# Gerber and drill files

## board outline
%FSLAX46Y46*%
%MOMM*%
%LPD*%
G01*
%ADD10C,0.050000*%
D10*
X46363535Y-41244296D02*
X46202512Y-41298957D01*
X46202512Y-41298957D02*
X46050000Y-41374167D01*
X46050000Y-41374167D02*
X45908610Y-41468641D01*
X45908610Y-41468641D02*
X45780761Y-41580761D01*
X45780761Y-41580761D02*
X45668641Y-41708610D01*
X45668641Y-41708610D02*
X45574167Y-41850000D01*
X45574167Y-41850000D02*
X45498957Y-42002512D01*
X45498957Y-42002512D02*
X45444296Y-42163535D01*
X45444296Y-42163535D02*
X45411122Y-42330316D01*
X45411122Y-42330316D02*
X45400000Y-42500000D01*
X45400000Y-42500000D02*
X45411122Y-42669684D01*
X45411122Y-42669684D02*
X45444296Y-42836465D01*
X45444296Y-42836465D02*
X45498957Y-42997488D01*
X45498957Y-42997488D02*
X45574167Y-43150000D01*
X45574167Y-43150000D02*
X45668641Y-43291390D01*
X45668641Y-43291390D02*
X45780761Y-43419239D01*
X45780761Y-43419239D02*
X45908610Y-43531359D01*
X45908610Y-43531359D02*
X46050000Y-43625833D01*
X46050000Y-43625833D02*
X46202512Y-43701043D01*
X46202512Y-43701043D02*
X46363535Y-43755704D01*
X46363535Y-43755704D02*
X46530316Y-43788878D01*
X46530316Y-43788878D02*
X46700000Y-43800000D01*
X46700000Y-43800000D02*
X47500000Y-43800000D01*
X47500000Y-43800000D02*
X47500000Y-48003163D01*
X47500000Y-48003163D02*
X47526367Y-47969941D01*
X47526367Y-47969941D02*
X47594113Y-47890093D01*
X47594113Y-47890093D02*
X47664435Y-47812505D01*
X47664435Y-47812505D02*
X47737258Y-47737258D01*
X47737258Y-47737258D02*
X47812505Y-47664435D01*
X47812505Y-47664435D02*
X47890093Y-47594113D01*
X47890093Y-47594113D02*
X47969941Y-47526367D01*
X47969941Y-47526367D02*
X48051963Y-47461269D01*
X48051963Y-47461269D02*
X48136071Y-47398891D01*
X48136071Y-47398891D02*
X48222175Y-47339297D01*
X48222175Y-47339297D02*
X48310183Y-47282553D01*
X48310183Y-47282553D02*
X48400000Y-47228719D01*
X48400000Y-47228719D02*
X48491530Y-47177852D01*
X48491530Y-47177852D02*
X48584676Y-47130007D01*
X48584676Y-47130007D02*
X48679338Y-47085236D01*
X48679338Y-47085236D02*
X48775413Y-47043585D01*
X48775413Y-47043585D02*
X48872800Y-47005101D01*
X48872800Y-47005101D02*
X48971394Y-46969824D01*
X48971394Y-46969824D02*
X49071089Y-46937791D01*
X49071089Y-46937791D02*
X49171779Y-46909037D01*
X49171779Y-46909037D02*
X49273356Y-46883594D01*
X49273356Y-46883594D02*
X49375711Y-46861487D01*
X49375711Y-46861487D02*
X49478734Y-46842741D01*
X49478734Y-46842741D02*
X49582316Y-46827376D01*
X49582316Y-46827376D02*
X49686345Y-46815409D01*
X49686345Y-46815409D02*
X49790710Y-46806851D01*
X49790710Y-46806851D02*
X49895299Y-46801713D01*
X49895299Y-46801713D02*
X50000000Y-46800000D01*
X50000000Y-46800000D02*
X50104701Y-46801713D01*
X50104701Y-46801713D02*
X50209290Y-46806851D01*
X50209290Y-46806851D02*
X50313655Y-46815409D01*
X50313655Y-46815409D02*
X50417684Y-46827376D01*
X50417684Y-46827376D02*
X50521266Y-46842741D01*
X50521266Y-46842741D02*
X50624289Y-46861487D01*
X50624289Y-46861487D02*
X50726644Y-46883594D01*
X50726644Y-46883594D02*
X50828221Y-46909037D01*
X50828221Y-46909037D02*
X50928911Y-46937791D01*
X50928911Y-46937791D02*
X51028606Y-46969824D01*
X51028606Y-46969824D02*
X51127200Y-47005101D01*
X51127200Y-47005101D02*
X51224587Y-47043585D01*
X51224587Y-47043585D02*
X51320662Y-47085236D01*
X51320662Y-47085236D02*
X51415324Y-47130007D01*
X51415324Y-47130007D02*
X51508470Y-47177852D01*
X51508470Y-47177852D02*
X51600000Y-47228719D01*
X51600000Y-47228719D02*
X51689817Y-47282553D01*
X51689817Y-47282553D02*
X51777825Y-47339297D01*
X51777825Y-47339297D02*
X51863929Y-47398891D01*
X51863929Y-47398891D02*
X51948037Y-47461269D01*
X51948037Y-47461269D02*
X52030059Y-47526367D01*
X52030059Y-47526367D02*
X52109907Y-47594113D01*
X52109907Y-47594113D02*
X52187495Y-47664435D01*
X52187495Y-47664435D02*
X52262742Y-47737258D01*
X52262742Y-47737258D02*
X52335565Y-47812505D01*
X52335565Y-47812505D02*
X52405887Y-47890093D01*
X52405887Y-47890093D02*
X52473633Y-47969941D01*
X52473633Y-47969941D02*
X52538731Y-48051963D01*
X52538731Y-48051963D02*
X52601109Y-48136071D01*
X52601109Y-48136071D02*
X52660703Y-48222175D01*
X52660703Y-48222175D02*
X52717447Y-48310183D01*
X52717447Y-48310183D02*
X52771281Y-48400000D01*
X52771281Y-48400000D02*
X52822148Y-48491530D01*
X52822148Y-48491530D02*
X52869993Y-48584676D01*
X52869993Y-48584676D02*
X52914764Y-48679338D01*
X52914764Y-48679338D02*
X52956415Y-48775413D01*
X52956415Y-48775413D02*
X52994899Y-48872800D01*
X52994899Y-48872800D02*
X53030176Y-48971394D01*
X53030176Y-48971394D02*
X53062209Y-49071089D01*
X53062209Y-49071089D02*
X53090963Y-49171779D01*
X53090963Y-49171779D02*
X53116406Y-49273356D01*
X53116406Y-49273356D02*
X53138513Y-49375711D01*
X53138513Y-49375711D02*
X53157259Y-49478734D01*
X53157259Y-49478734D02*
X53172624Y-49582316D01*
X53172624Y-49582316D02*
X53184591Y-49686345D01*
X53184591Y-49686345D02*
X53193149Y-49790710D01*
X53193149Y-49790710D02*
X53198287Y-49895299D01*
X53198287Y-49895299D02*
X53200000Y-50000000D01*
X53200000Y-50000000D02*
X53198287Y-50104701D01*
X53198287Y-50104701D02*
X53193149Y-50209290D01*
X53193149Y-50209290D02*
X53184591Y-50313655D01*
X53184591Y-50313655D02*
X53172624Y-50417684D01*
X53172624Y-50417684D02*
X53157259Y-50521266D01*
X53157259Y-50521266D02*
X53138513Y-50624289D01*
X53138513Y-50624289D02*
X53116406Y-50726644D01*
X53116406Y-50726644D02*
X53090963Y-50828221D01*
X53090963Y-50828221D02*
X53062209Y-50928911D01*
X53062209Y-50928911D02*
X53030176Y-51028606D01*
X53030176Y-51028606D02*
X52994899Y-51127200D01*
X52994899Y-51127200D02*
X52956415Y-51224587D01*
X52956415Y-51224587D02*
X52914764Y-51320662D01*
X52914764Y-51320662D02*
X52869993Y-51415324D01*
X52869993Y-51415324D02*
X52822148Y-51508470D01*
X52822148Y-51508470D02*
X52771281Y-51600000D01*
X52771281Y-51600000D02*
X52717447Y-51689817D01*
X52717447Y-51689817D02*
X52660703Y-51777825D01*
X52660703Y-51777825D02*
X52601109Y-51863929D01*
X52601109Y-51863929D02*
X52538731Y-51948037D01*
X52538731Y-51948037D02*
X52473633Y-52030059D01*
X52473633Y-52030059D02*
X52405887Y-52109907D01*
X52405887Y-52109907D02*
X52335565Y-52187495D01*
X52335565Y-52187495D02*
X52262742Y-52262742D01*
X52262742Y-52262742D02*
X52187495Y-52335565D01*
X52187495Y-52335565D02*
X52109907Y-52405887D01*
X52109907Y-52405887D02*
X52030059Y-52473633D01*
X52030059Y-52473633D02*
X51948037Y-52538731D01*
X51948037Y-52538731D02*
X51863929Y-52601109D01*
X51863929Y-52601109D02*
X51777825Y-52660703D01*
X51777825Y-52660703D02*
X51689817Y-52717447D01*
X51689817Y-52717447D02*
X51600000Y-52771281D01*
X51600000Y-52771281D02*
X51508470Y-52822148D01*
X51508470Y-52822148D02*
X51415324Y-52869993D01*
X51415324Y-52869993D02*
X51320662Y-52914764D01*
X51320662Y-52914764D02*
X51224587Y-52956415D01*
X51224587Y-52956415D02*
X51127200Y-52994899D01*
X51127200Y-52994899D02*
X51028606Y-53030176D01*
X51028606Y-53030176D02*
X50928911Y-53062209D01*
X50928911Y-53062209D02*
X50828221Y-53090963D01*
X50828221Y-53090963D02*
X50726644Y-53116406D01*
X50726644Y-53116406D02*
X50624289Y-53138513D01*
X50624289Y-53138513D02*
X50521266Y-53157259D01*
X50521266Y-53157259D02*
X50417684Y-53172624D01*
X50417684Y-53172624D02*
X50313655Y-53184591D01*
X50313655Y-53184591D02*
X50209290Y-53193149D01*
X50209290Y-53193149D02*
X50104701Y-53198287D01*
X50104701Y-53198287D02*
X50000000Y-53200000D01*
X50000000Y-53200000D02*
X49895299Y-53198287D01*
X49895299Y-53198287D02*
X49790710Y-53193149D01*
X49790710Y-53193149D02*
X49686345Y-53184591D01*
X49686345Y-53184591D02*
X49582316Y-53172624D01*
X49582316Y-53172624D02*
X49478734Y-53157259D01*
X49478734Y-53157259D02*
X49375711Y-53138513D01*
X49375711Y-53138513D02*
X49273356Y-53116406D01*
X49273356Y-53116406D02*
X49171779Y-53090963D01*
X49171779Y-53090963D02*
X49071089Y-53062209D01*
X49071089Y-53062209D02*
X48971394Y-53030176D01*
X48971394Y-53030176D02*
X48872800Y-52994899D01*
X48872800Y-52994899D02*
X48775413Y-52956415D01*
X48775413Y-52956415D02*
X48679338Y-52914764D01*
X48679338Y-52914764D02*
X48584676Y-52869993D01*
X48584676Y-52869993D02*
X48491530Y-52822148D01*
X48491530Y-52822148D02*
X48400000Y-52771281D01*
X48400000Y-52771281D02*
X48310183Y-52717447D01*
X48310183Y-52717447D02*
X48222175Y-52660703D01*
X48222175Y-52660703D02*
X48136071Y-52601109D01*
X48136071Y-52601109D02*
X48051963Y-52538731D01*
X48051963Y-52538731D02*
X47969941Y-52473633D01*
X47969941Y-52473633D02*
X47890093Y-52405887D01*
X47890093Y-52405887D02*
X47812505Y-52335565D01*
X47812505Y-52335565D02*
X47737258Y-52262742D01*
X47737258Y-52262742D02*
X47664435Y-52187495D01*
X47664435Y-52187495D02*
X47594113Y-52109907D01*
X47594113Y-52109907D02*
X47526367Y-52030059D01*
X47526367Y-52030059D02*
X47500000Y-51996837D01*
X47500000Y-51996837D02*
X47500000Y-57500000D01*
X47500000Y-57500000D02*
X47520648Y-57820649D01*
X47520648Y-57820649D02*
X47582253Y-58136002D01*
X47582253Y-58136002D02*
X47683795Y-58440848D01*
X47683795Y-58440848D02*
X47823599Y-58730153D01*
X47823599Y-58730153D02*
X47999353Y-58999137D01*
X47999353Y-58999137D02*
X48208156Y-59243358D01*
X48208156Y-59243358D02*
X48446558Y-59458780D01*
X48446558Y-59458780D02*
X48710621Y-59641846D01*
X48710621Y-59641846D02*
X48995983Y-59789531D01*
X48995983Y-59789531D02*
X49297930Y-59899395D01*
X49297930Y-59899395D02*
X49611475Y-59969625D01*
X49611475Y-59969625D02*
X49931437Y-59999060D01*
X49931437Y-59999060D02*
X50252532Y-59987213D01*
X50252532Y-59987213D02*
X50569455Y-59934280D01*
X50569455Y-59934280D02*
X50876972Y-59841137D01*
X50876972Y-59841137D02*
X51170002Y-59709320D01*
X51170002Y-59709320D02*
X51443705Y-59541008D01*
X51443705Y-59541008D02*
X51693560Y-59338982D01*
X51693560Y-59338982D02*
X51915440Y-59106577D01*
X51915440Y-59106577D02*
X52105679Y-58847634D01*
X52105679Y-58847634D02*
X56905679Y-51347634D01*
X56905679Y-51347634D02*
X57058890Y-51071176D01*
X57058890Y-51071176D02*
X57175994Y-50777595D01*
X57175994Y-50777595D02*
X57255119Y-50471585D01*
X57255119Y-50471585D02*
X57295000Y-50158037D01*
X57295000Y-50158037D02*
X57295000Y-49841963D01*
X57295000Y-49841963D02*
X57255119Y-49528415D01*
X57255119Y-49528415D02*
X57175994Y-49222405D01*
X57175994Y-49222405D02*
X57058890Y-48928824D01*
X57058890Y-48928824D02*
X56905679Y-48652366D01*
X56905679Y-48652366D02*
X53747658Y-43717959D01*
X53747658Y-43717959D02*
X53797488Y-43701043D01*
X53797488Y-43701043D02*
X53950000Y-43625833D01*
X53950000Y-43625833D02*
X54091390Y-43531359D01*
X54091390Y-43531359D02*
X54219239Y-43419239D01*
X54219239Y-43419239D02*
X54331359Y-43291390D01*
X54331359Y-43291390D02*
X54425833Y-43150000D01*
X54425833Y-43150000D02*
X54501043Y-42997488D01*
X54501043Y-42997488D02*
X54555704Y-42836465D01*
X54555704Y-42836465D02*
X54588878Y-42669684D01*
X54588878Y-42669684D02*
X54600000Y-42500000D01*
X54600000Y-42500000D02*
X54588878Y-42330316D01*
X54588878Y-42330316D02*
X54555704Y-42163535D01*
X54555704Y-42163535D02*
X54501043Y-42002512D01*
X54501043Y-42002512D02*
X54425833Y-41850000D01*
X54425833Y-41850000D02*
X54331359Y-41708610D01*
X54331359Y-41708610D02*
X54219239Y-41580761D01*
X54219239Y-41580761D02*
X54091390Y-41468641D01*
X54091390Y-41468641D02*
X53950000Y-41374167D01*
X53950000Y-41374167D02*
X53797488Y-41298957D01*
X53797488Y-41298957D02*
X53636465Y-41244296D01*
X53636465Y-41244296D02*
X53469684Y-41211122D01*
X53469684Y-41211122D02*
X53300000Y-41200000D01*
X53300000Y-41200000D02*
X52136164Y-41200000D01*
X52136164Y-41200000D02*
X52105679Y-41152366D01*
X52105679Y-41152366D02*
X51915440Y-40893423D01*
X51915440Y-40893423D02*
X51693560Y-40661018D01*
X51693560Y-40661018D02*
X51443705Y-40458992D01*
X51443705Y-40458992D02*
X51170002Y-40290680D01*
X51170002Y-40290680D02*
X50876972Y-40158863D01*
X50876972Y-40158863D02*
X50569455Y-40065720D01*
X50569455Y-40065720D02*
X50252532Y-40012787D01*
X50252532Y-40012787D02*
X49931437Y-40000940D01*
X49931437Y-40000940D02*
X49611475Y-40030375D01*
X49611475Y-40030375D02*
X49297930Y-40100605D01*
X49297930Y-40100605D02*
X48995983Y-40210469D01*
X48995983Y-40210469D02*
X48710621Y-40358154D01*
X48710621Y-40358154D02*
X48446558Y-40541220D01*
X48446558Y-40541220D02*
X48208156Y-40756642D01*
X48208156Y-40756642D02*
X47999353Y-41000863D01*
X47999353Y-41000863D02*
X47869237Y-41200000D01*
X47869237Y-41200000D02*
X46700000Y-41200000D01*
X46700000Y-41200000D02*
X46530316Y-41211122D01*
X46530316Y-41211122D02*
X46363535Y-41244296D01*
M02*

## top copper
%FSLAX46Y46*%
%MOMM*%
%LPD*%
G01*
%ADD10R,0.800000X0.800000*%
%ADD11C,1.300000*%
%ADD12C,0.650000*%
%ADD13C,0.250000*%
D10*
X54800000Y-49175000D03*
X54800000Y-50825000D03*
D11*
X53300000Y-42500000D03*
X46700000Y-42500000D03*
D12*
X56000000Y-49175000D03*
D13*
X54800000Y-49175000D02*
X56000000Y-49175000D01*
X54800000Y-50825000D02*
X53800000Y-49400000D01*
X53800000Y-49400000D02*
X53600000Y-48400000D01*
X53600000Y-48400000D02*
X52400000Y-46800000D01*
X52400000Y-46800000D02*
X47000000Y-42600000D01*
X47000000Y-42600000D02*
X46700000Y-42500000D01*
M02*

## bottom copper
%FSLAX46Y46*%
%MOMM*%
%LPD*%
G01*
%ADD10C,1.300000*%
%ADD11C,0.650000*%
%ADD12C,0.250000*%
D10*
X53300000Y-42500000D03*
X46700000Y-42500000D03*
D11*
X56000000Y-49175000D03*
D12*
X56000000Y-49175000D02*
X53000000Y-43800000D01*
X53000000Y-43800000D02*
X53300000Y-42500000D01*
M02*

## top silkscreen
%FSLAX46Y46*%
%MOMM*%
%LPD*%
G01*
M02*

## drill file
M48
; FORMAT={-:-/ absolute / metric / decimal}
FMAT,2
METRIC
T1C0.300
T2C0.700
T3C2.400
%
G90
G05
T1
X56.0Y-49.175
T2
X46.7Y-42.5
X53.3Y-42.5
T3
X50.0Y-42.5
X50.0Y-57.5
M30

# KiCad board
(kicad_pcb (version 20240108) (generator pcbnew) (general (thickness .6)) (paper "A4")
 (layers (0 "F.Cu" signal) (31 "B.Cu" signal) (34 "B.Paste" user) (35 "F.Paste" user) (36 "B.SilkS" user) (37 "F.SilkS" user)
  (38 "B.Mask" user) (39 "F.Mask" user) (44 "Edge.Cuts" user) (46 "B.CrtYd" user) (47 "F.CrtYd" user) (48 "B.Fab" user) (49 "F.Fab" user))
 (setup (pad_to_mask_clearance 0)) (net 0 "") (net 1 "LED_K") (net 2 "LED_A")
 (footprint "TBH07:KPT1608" (layer "F.Cu") (at 54.8 50)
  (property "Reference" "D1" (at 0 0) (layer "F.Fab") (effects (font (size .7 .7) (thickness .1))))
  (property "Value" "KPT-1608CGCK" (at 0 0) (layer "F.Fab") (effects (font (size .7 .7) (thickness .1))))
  (pad "1" smd rect (at 0 -.825) (size .8 .8) (layers "F.Cu" "F.Paste" "F.Mask") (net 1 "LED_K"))
  (pad "2" smd rect (at 0 .825) (size .8 .8) (layers "F.Cu" "F.Paste" "F.Mask") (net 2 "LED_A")))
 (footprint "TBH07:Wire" (layer "F.Cu") (at 53.3 42.5)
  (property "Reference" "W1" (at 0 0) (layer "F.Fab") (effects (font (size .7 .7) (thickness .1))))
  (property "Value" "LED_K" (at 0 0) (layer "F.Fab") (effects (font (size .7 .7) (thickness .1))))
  (pad "1" thru_hole circle (at 0 0) (size 1.3 1.3) (drill .7) (layers "*.Cu" "*.Mask") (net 1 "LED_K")))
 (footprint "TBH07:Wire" (layer "F.Cu") (at 46.7 42.5)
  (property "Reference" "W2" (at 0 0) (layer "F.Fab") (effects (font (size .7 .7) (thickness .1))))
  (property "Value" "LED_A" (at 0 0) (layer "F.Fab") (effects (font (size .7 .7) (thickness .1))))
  (pad "1" thru_hole circle (at 0 0) (size 1.3 1.3) (drill .7) (layers "*.Cu" "*.Mask") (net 2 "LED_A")))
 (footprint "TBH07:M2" (layer "F.Cu") (at 50 42.5)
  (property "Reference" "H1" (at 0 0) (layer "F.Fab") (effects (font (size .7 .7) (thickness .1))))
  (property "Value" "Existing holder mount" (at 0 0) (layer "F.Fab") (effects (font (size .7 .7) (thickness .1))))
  (pad "" np_thru_hole circle (at 0 0) (size 2.4 2.4) (drill 2.4) (layers "*.Cu" "*.Mask")))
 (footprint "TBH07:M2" (layer "F.Cu") (at 50 57.5)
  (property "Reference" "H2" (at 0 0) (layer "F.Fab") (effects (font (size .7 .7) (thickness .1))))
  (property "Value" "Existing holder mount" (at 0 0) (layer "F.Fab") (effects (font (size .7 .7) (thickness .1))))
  (pad "" np_thru_hole circle (at 0 0) (size 2.4 2.4) (drill 2.4) (layers "*.Cu" "*.Mask")))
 (segment (start 54.8 49.175) (end 56 49.175) (width .25) (layer "F.Cu") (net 1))
 (via (at 56 49.175) (size .65) (drill .3) (layers "F.Cu" "B.Cu") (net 1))
 (segment (start 56 49.175) (end 53.0 43.8) (width .25) (layer "B.Cu") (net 1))
 (segment (start 53.0 43.8) (end 53.3 42.5) (width .25) (layer "B.Cu") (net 1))
 (segment (start 54.8 50.825) (end 53.8 49.4) (width .25) (layer "F.Cu") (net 2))
 (segment (start 53.8 49.4) (end 53.6 48.4) (width .25) (layer "F.Cu") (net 2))
 (segment (start 53.6 48.4) (end 52.4 46.8) (width .25) (layer "F.Cu") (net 2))
 (segment (start 52.4 46.8) (end 47.0 42.6) (width .25) (layer "F.Cu") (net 2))
 (segment (start 47.0 42.6) (end 46.7 42.5) (width .25) (layer "F.Cu") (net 2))
 (gr_line (start 46.363535241366726 41.24429642582421) (end 46.20251153792538 41.29895660773533) (stroke (width .05) (type default))
  (layer "Edge.Cuts"))
 (gr_line (start 46.20251153792538 41.29895660773533) (end 46.05 41.37416697508023) (stroke (width .05) (type default)) (layer "Edge.Cuts"))
 (gr_line (start 46.05 41.37416697508023) (end 45.908610142288666 41.46864065762139) (stroke (width .05) (type default)) (layer "Edge.Cuts"))
 (gr_line (start 45.908610142288666 41.46864065762139) (end 45.78076118445749 41.58076118445749) (stroke (width .05) (type default))
  (layer "Edge.Cuts"))
 (gr_line (start 45.78076118445749 41.58076118445749) (end 45.668640657621395 41.70861014228866) (stroke (width .05) (type default))
  (layer "Edge.Cuts"))
 (gr_line (start 45.668640657621395 41.70861014228866) (end 45.57416697508023 41.85) (stroke (width .05) (type default)) (layer "Edge.Cuts"))
 (gr_line (start 45.57416697508023 41.85) (end 45.49895660773532 42.002511537925386) (stroke (width .05) (type default)) (layer "Edge.Cuts"))
 (gr_line (start 45.49895660773532 42.002511537925386) (end 45.44429642582421 42.16353524136672) (stroke (width .05) (type default))
  (layer "Edge.Cuts"))
 (gr_line (start 45.44429642582421 42.16353524136672) (end 45.411121680214045 42.330315950113935) (stroke (width .05) (type default))
  (layer "Edge.Cuts"))
 (gr_line (start 45.411121680214045 42.330315950113935) (end 45.4 42.5) (stroke (width .05) (type default)) (layer "Edge.Cuts"))
 (gr_line (start 45.4 42.5) (end 45.411121680214045 42.669684049886065) (stroke (width .05) (type default)) (layer "Edge.Cuts"))
 (gr_line (start 45.411121680214045 42.669684049886065) (end 45.44429642582421 42.83646475863328) (stroke (width .05) (type default))
  (layer "Edge.Cuts"))
 (gr_line (start 45.44429642582421 42.83646475863328) (end 45.49895660773532 42.997488462074614) (stroke (width .05) (type default))
  (layer "Edge.Cuts"))
 (gr_line (start 45.49895660773532 42.997488462074614) (end 45.57416697508023 43.15) (stroke (width .05) (type default)) (layer "Edge.Cuts"))
 (gr_line (start 45.57416697508023 43.15) (end 45.668640657621395 43.29138985771134) (stroke (width .05) (type default)) (layer "Edge.Cuts"))
 (gr_line (start 45.668640657621395 43.29138985771134) (end 45.78076118445749 43.41923881554251) (stroke (width .05) (type default))
  (layer "Edge.Cuts"))
 (gr_line (start 45.78076118445749 43.41923881554251) (end 45.908610142288666 43.53135934237861) (stroke (width .05) (type default))
  (layer "Edge.Cuts"))
 (gr_line (start 45.908610142288666 43.53135934237861) (end 46.05 43.62583302491977) (stroke (width .05) (type default)) (layer "Edge.Cuts"))
 (gr_line (start 46.05 43.62583302491977) (end 46.20251153792538 43.70104339226467) (stroke (width .05) (type default)) (layer "Edge.Cuts"))
 (gr_line (start 46.20251153792538 43.70104339226467) (end 46.363535241366726 43.75570357417579) (stroke (width .05) (type default))
  (layer "Edge.Cuts"))
 (gr_line (start 46.363535241366726 43.75570357417579) (end 46.53031595011393 43.78887831978595) (stroke (width .05) (type default))
  (layer "Edge.Cuts"))
 (gr_line (start 46.53031595011393 43.78887831978595) (end 46.7 43.8) (stroke (width .05) (type default)) (layer "Edge.Cuts"))
 (gr_line (start 46.7 43.8) (end 47.5 43.8) (stroke (width .05) (type default)) (layer "Edge.Cuts"))
 (gr_line (start 47.5 43.8) (end 47.5 48.00316310634037) (stroke (width .05) (type default)) (layer "Edge.Cuts"))
 (gr_line (start 47.5 48.00316310634037) (end 47.52636654923924 47.969941490676334) (stroke (width .05) (type default)) (layer "Edge.Cuts"))
 (gr_line (start 47.52636654923924 47.969941490676334) (end 47.59411261606727 47.89009339167978) (stroke (width .05) (type default))
  (layer "Edge.Cuts"))
 (gr_line (start 47.59411261606727 47.89009339167978) (end 47.66443496736693 47.812504633526814) (stroke (width .05) (type default))
  (layer "Edge.Cuts"))
 (gr_line (start 47.66443496736693 47.812504633526814) (end 47.737258300203045 47.737258300203045) (stroke (width .05) (type default))
  (layer "Edge.Cuts"))
 (gr_line (start 47.737258300203045 47.737258300203045) (end 47.812504633526814 47.66443496736692) (stroke (width .05) (type default))
  (layer "Edge.Cuts"))
 (gr_line (start 47.812504633526814 47.66443496736692) (end 47.890093391679784 47.59411261606727) (stroke (width .05) (type default))
  (layer "Edge.Cuts"))
 (gr_line (start 47.890093391679784 47.59411261606727) (end 47.969941490676334 47.52636654923924) (stroke (width .05) (type default))
  (layer "Edge.Cuts"))
 (gr_line (start 47.969941490676334 47.52636654923924) (end 48.0519634271721 47.461269311068044) (stroke (width .05) (type default))
  (layer "Edge.Cuts"))
 (gr_line (start 48.0519634271721 47.461269311068044) (end 48.13607137002303 47.39889060930683) (stroke (width .05) (type default))
  (layer "Edge.Cuts"))
 (gr_line (start 48.13607137002303 47.39889060930683) (end 48.22217525433727 47.33929724063186) (stroke (width .05) (type default))
  (layer "Edge.Cuts"))
 (gr_line (start 48.22217525433727 47.33929724063186) (end 48.31018287791882 47.28255301911495) (stroke (width .05) (type default))
  (layer "Edge.Cuts"))
 (gr_line (start 48.31018287791882 47.28255301911495) (end 48.4 47.2287187078898) (stroke (width .05) (type default)) (layer "Edge.Cuts"))
 (gr_line (start 48.4 47.2287187078898) (end 48.49153044215681 47.17785195408526) (stroke (width .05) (type default)) (layer "Edge.Cuts"))
 (gr_line (start 48.49153044215681 47.17785195408526) (end 48.584676191299195 47.1300072270954) (stroke (width .05) (type default))
  (layer "Edge.Cuts"))
 (gr_line (start 48.584676191299195 47.1300072270954) (end 48.679337504625934 47.08523576025224) (stroke (width .05) (type default))
  (layer "Edge.Cuts"))
 (gr_line (start 48.679337504625934 47.08523576025224) (end 48.77541301643171 47.04358549596388) (stroke (width .05) (type default))
  (layer "Edge.Cuts"))
 (gr_line (start 48.77541301643171 47.04358549596388) (end 48.87279984665205 47.00510103437656) (stroke (width .05) (type default))
  (layer "Edge.Cuts"))
 (gr_line (start 48.87279984665205 47.00510103437656) (end 48.97139371102988 46.969823585615664) (stroke (width .05) (type default))
  (layer "Edge.Cuts"))
 (gr_line (start 48.97139371102988 46.969823585615664) (end 49.07108903278572 46.937790925656934) (stroke (width .05) (type default))
  (layer "Edge.Cuts"))
 (gr_line (start 49.07108903278572 46.937790925656934) (end 49.171779055671934 46.90903735587498) (stroke (width .05) (type default))
  (layer "Edge.Cuts"))
 (gr_line (start 49.171779055671934 46.90903735587498) (end 49.273355958290004 46.883593666312535) (stroke (width .05) (type default))
  (layer "Edge.Cuts"))
 (gr_line (start 49.273355958290004 46.883593666312535) (end 49.37571096954839 46.86148710270966) (stroke (width .05) (type default))
  (layer "Edge.Cuts"))
 (gr_line (start 49.37571096954839 46.86148710270966) (end 49.478734485137316 46.842741337328384) (stroke (width .05) (type default))
  (layer "Edge.Cuts"))
 (gr_line (start 49.478734485137316 46.842741337328384) (end 49.58231618489584 46.827376443603804) (stroke (width .05) (type default))
  (layer "Edge.Cuts"))
 (gr_line (start 49.58231618489584 46.827376443603804) (end 49.68634515094541 46.815408874648966) (stroke (width .05) (type default))
  (layer "Edge.Cuts"))
 (gr_line (start 49.68634515094541 46.815408874648966) (end 49.79070998646354 46.80685144563647) (stroke (width .05) (type default))
  (layer "Edge.Cuts"))
 (gr_line (start 49.79070998646354 46.80685144563647) (end 49.89529893497032 46.80171332007563) (stroke (width .05) (type default))
  (layer "Edge.Cuts"))
 (gr_line (start 49.89529893497032 46.80171332007563) (end 50.0 46.8) (stroke (width .05) (type default)) (layer "Edge.Cuts"))
 (gr_line (start 50.0 46.8) (end 50.10470106502969 46.80171332007563) (stroke (width .05) (type default)) (layer "Edge.Cuts"))
 (gr_line (start 50.10470106502969 46.80171332007563) (end 50.20929001353646 46.80685144563647) (stroke (width .05) (type default))
  (layer "Edge.Cuts"))
 (gr_line (start 50.20929001353646 46.80685144563647) (end 50.31365484905459 46.815408874648966) (stroke (width .05) (type default))
  (layer "Edge.Cuts"))
 (gr_line (start 50.31365484905459 46.815408874648966) (end 50.41768381510416 46.827376443603804) (stroke (width .05) (type default))
  (layer "Edge.Cuts"))
 (gr_line (start 50.41768381510416 46.827376443603804) (end 50.521265514862684 46.842741337328384) (stroke (width .05) (type default))
  (layer "Edge.Cuts"))
 (gr_line (start 50.521265514862684 46.842741337328384) (end 50.624289030451614 46.86148710270966) (stroke (width .05) (type default))
  (layer "Edge.Cuts"))
 (gr_line (start 50.624289030451614 46.86148710270966) (end 50.726644041709996 46.883593666312535) (stroke (width .05) (type default))
  (layer "Edge.Cuts"))
 (gr_line (start 50.726644041709996 46.883593666312535) (end 50.828220944328066 46.90903735587498) (stroke (width .05) (type default))
  (layer "Edge.Cuts"))
 (gr_line (start 50.828220944328066 46.90903735587498) (end 50.92891096721428 46.937790925656934) (stroke (width .05) (type default))
  (layer "Edge.Cuts"))
 (gr_line (start 50.92891096721428 46.937790925656934) (end 51.02860628897012 46.969823585615664) (stroke (width .05) (type default))
  (layer "Edge.Cuts"))
 (gr_line (start 51.02860628897012 46.969823585615664) (end 51.12720015334795 47.00510103437656) (stroke (width .05) (type default))
  (layer "Edge.Cuts"))
 (gr_line (start 51.12720015334795 47.00510103437656) (end 51.22458698356829 47.04358549596388) (stroke (width .05) (type default))
  (layer "Edge.Cuts"))
 (gr_line (start 51.22458698356829 47.04358549596388) (end 51.320662495374066 47.08523576025224) (stroke (width .05) (type default))
  (layer "Edge.Cuts"))
 (gr_line (start 51.320662495374066 47.08523576025224) (end 51.415323808700805 47.1300072270954) (stroke (width .05) (type default))
  (layer "Edge.Cuts"))
 (gr_line (start 51.415323808700805 47.1300072270954) (end 51.50846955784319 47.17785195408526) (stroke (width .05) (type default))
  (layer "Edge.Cuts"))
 (gr_line (start 51.50846955784319 47.17785195408526) (end 51.6 47.2287187078898) (stroke (width .05) (type default)) (layer "Edge.Cuts"))
 (gr_line (start 51.6 47.2287187078898) (end 51.68981712208118 47.28255301911495) (stroke (width .05) (type default)) (layer "Edge.Cuts"))
 (gr_line (start 51.68981712208118 47.28255301911495) (end 51.77782474566273 47.33929724063186) (stroke (width .05) (type default))
  (layer "Edge.Cuts"))
 (gr_line (start 51.77782474566273 47.33929724063186) (end 51.86392862997697 47.39889060930683) (stroke (width .05) (type default))
  (layer "Edge.Cuts"))
 (gr_line (start 51.86392862997697 47.39889060930683) (end 51.9480365728279 47.46126931106805) (stroke (width .05) (type default))
  (layer "Edge.Cuts"))
 (gr_line (start 51.9480365728279 47.46126931106805) (end 52.030058509323666 47.52636654923924) (stroke (width .05) (type default))
  (layer "Edge.Cuts"))
 (gr_line (start 52.030058509323666 47.52636654923924) (end 52.10990660832022 47.59411261606727) (stroke (width .05) (type default))
  (layer "Edge.Cuts"))
 (gr_line (start 52.10990660832022 47.59411261606727) (end 52.187495366473186 47.66443496736693) (stroke (width .05) (type default))
  (layer "Edge.Cuts"))
 (gr_line (start 52.187495366473186 47.66443496736693) (end 52.262741699796955 47.737258300203045) (stroke (width .05) (type default))
  (layer "Edge.Cuts"))
 (gr_line (start 52.262741699796955 47.737258300203045) (end 52.33556503263308 47.812504633526814) (stroke (width .05) (type default))
  (layer "Edge.Cuts"))
 (gr_line (start 52.33556503263308 47.812504633526814) (end 52.40588738393273 47.89009339167978) (stroke (width .05) (type default))
  (layer "Edge.Cuts"))
 (gr_line (start 52.40588738393273 47.89009339167978) (end 52.47363345076076 47.969941490676334) (stroke (width .05) (type default))
  (layer "Edge.Cuts"))
 (gr_line (start 52.47363345076076 47.969941490676334) (end 52.538730688931956 48.0519634271721) (stroke (width .05) (type default))
  (layer "Edge.Cuts"))
 (gr_line (start 52.538730688931956 48.0519634271721) (end 52.60110939069317 48.13607137002303) (stroke (width .05) (type default))
  (layer "Edge.Cuts"))
 (gr_line (start 52.60110939069317 48.13607137002303) (end 52.66070275936814 48.22217525433727) (stroke (width .05) (type default))
  (layer "Edge.Cuts"))
 (gr_line (start 52.66070275936814 48.22217525433727) (end 52.71744698088505 48.31018287791882) (stroke (width .05) (type default))
  (layer "Edge.Cuts"))
 (gr_line (start 52.71744698088505 48.31018287791882) (end 52.7712812921102 48.4) (stroke (width .05) (type default)) (layer "Edge.Cuts"))
 (gr_line (start 52.7712812921102 48.4) (end 52.82214804591474 48.49153044215681) (stroke (width .05) (type default)) (layer "Edge.Cuts"))
 (gr_line (start 52.82214804591474 48.49153044215681) (end 52.8699927729046 48.584676191299195) (stroke (width .05) (type default))
  (layer "Edge.Cuts"))
 (gr_line (start 52.8699927729046 48.584676191299195) (end 52.91476423974776 48.679337504625934) (stroke (width .05) (type default))
  (layer "Edge.Cuts"))
 (gr_line (start 52.91476423974776 48.679337504625934) (end 52.95641450403612 48.77541301643171) (stroke (width .05) (type default))
  (layer "Edge.Cuts"))
 (gr_line (start 52.95641450403612 48.77541301643171) (end 52.99489896562344 48.87279984665205) (stroke (width .05) (type default))
  (layer "Edge.Cuts"))
 (gr_line (start 52.99489896562344 48.87279984665205) (end 53.030176414384336 48.97139371102988) (stroke (width .05) (type default))
  (layer "Edge.Cuts"))
 (gr_line (start 53.030176414384336 48.97139371102988) (end 53.062209074343066 49.07108903278572) (stroke (width .05) (type default))
  (layer "Edge.Cuts"))
 (gr_line (start 53.062209074343066 49.07108903278572) (end 53.09096264412502 49.171779055671934) (stroke (width .05) (type default))
  (layer "Edge.Cuts"))
 (gr_line (start 53.09096264412502 49.171779055671934) (end 53.116406333687465 49.273355958290004) (stroke (width .05) (type default))
  (layer "Edge.Cuts"))
 (gr_line (start 53.116406333687465 49.273355958290004) (end 53.13851289729034 49.375710969548386) (stroke (width .05) (type default))
  (layer "Edge.Cuts"))
 (gr_line (start 53.13851289729034 49.375710969548386) (end 53.157258662671616 49.478734485137316) (stroke (width .05) (type default))
  (layer "Edge.Cuts"))
 (gr_line (start 53.157258662671616 49.478734485137316) (end 53.172623556396196 49.58231618489584) (stroke (width .05) (type default))
  (layer "Edge.Cuts"))
 (gr_line (start 53.172623556396196 49.58231618489584) (end 53.184591125351034 49.68634515094541) (stroke (width .05) (type default))
  (layer "Edge.Cuts"))
 (gr_line (start 53.184591125351034 49.68634515094541) (end 53.19314855436353 49.79070998646354) (stroke (width .05) (type default))
  (layer "Edge.Cuts"))
 (gr_line (start 53.19314855436353 49.79070998646354) (end 53.19828667992437 49.89529893497031) (stroke (width .05) (type default))
  (layer "Edge.Cuts"))
 (gr_line (start 53.19828667992437 49.89529893497031) (end 53.2 50.0) (stroke (width .05) (type default)) (layer "Edge.Cuts"))
 (gr_line (start 53.2 50.0) (end 53.19828667992437 50.10470106502969) (stroke (width .05) (type default)) (layer "Edge.Cuts"))
 (gr_line (start 53.19828667992437 50.10470106502969) (end 53.19314855436353 50.20929001353646) (stroke (width .05) (type default))
  (layer "Edge.Cuts"))
 (gr_line (start 53.19314855436353 50.20929001353646) (end 53.184591125351034 50.31365484905459) (stroke (width .05) (type default))
  (layer "Edge.Cuts"))
 (gr_line (start 53.184591125351034 50.31365484905459) (end 53.17262355639619 50.41768381510417) (stroke (width .05) (type default))
  (layer "Edge.Cuts"))
 (gr_line (start 53.17262355639619 50.41768381510417) (end 53.157258662671616 50.521265514862684) (stroke (width .05) (type default))
  (layer "Edge.Cuts"))
 (gr_line (start 53.157258662671616 50.521265514862684) (end 53.13851289729034 50.624289030451614) (stroke (width .05) (type default))
  (layer "Edge.Cuts"))
 (gr_line (start 53.13851289729034 50.624289030451614) (end 53.116406333687465 50.726644041709996) (stroke (width .05) (type default))
  (layer "Edge.Cuts"))
 (gr_line (start 53.116406333687465 50.726644041709996) (end 53.09096264412502 50.828220944328066) (stroke (width .05) (type default))
  (layer "Edge.Cuts"))
 (gr_line (start 53.09096264412502 50.828220944328066) (end 53.062209074343066 50.928910967214286) (stroke (width .05) (type default))
  (layer "Edge.Cuts"))
 (gr_line (start 53.062209074343066 50.928910967214286) (end 53.030176414384336 51.02860628897012) (stroke (width .05) (type default))
  (layer "Edge.Cuts"))
 (gr_line (start 53.030176414384336 51.02860628897012) (end 52.99489896562344 51.12720015334795) (stroke (width .05) (type default))
  (layer "Edge.Cuts"))
 (gr_line (start 52.99489896562344 51.12720015334795) (end 52.95641450403612 51.22458698356829) (stroke (width .05) (type default))
  (layer "Edge.Cuts"))
 (gr_line (start 52.95641450403612 51.22458698356829) (end 52.91476423974776 51.320662495374066) (stroke (width .05) (type default))
  (layer "Edge.Cuts"))
 (gr_line (start 52.91476423974776 51.320662495374066) (end 52.8699927729046 51.415323808700805) (stroke (width .05) (type default))
  (layer "Edge.Cuts"))
 (gr_line (start 52.8699927729046 51.415323808700805) (end 52.82214804591474 51.50846955784319) (stroke (width .05) (type default))
  (layer "Edge.Cuts"))
 (gr_line (start 52.82214804591474 51.50846955784319) (end 52.7712812921102 51.6) (stroke (width .05) (type default)) (layer "Edge.Cuts"))
 (gr_line (start 52.7712812921102 51.6) (end 52.71744698088505 51.68981712208118) (stroke (width .05) (type default)) (layer "Edge.Cuts"))
 (gr_line (start 52.71744698088505 51.68981712208118) (end 52.66070275936814 51.77782474566273) (stroke (width .05) (type default))
  (layer "Edge.Cuts"))
 (gr_line (start 52.66070275936814 51.77782474566273) (end 52.60110939069317 51.86392862997697) (stroke (width .05) (type default))
  (layer "Edge.Cuts"))
 (gr_line (start 52.60110939069317 51.86392862997697) (end 52.53873068893195 51.94803657282791) (stroke (width .05) (type default))
  (layer "Edge.Cuts"))
 (gr_line (start 52.53873068893195 51.94803657282791) (end 52.47363345076076 52.030058509323666) (stroke (width .05) (type default))
  (layer "Edge.Cuts"))
 (gr_line (start 52.47363345076076 52.030058509323666) (end 52.40588738393273 52.10990660832022) (stroke (width .05) (type default))
  (layer "Edge.Cuts"))
 (gr_line (start 52.40588738393273 52.10990660832022) (end 52.33556503263307 52.18749536647319) (stroke (width .05) (type default))
  (layer "Edge.Cuts"))
 (gr_line (start 52.33556503263307 52.18749536647319) (end 52.262741699796955 52.262741699796955) (stroke (width .05) (type default))
  (layer "Edge.Cuts"))
 (gr_line (start 52.262741699796955 52.262741699796955) (end 52.187495366473186 52.33556503263308) (stroke (width .05) (type default))
  (layer "Edge.Cuts"))
 (gr_line (start 52.187495366473186 52.33556503263308) (end 52.109906608320216 52.40588738393273) (stroke (width .05) (type default))
  (layer "Edge.Cuts"))
 (gr_line (start 52.109906608320216 52.40588738393273) (end 52.030058509323666 52.47363345076076) (stroke (width .05) (type default))
  (layer "Edge.Cuts"))
 (gr_line (start 52.030058509323666 52.47363345076076) (end 51.9480365728279 52.538730688931956) (stroke (width .05) (type default))
  (layer "Edge.Cuts"))
 (gr_line (start 51.9480365728279 52.538730688931956) (end 51.86392862997697 52.60110939069317) (stroke (width .05) (type default))
  (layer "Edge.Cuts"))
 (gr_line (start 51.86392862997697 52.60110939069317) (end 51.77782474566273 52.66070275936815) (stroke (width .05) (type default))
  (layer "Edge.Cuts"))
 (gr_line (start 51.77782474566273 52.66070275936815) (end 51.68981712208117 52.71744698088506) (stroke (width .05) (type default))
  (layer "Edge.Cuts"))
 (gr_line (start 51.68981712208117 52.71744698088506) (end 51.599999999999994 52.7712812921102) (stroke (width .05) (type default))
  (layer "Edge.Cuts"))
 (gr_line (start 51.599999999999994 52.7712812921102) (end 51.50846955784319 52.82214804591474) (stroke (width .05) (type default))
  (layer "Edge.Cuts"))
 (gr_line (start 51.50846955784319 52.82214804591474) (end 51.415323808700805 52.8699927729046) (stroke (width .05) (type default))
  (layer "Edge.Cuts"))
 (gr_line (start 51.415323808700805 52.8699927729046) (end 51.32066249537406 52.91476423974776) (stroke (width .05) (type default))
  (layer "Edge.Cuts"))
 (gr_line (start 51.32066249537406 52.91476423974776) (end 51.22458698356829 52.95641450403612) (stroke (width .05) (type default))
  (layer "Edge.Cuts"))
 (gr_line (start 51.22458698356829 52.95641450403612) (end 51.12720015334794 52.99489896562344) (stroke (width .05) (type default))
  (layer "Edge.Cuts"))
 (gr_line (start 51.12720015334794 52.99489896562344) (end 51.02860628897012 53.030176414384336) (stroke (width .05) (type default))
  (layer "Edge.Cuts"))
 (gr_line (start 51.02860628897012 53.030176414384336) (end 50.92891096721428 53.062209074343066) (stroke (width .05) (type default))
  (layer "Edge.Cuts"))
 (gr_line (start 50.92891096721428 53.062209074343066) (end 50.828220944328066 53.09096264412502) (stroke (width .05) (type default))
  (layer "Edge.Cuts"))
 (gr_line (start 50.828220944328066 53.09096264412502) (end 50.72664404170999 53.116406333687465) (stroke (width .05) (type default))
  (layer "Edge.Cuts"))
 (gr_line (start 50.72664404170999 53.116406333687465) (end 50.62428903045161 53.13851289729034) (stroke (width .05) (type default))
  (layer "Edge.Cuts"))
 (gr_line (start 50.62428903045161 53.13851289729034) (end 50.521265514862684 53.157258662671616) (stroke (width .05) (type default))
  (layer "Edge.Cuts"))
 (gr_line (start 50.521265514862684 53.157258662671616) (end 50.41768381510416 53.172623556396196) (stroke (width .05) (type default))
  (layer "Edge.Cuts"))
 (gr_line (start 50.41768381510416 53.172623556396196) (end 50.31365484905459 53.184591125351034) (stroke (width .05) (type default))
  (layer "Edge.Cuts"))
 (gr_line (start 50.31365484905459 53.184591125351034) (end 50.20929001353645 53.19314855436353) (stroke (width .05) (type default))
  (layer "Edge.Cuts"))
 (gr_line (start 50.20929001353645 53.19314855436353) (end 50.10470106502968 53.19828667992437) (stroke (width .05) (type default))
  (layer "Edge.Cuts"))
 (gr_line (start 50.10470106502968 53.19828667992437) (end 50.0 53.2) (stroke (width .05) (type default)) (layer "Edge.Cuts"))
 (gr_line (start 50.0 53.2) (end 49.89529893497031 53.19828667992437) (stroke (width .05) (type default)) (layer "Edge.Cuts"))
 (gr_line (start 49.89529893497031 53.19828667992437) (end 49.79070998646354 53.19314855436353) (stroke (width .05) (type default))
  (layer "Edge.Cuts"))
 (gr_line (start 49.79070998646354 53.19314855436353) (end 49.68634515094541 53.184591125351034) (stroke (width .05) (type default))
  (layer "Edge.Cuts"))
 (gr_line (start 49.68634515094541 53.184591125351034) (end 49.58231618489583 53.17262355639619) (stroke (width .05) (type default))
  (layer "Edge.Cuts"))
 (gr_line (start 49.58231618489583 53.17262355639619) (end 49.478734485137316 53.157258662671616) (stroke (width .05) (type default))
  (layer "Edge.Cuts"))
 (gr_line (start 49.478734485137316 53.157258662671616) (end 49.375710969548386 53.13851289729034) (stroke (width .05) (type default))
  (layer "Edge.Cuts"))
 (gr_line (start 49.375710969548386 53.13851289729034) (end 49.273355958290004 53.116406333687465) (stroke (width .05) (type default))
  (layer "Edge.Cuts"))
 (gr_line (start 49.273355958290004 53.116406333687465) (end 49.171779055671934 53.09096264412502) (stroke (width .05) (type default))
  (layer "Edge.Cuts"))
 (gr_line (start 49.171779055671934 53.09096264412502) (end 49.07108903278572 53.062209074343066) (stroke (width .05) (type default))
  (layer "Edge.Cuts"))
 (gr_line (start 49.07108903278572 53.062209074343066) (end 48.97139371102988 53.030176414384336) (stroke (width .05) (type default))
  (layer "Edge.Cuts"))
 (gr_line (start 48.97139371102988 53.030176414384336) (end 48.87279984665205 52.99489896562344) (stroke (width .05) (type default))
  (layer "Edge.Cuts"))
 (gr_line (start 48.87279984665205 52.99489896562344) (end 48.77541301643171 52.95641450403612) (stroke (width .05) (type default))
  (layer "Edge.Cuts"))
 (gr_line (start 48.77541301643171 52.95641450403612) (end 48.679337504625934 52.91476423974776) (stroke (width .05) (type default))
  (layer "Edge.Cuts"))
 (gr_line (start 48.679337504625934 52.91476423974776) (end 48.584676191299195 52.8699927729046) (stroke (width .05) (type default))
  (layer "Edge.Cuts"))
 (gr_line (start 48.584676191299195 52.8699927729046) (end 48.49153044215681 52.82214804591474) (stroke (width .05) (type default))
  (layer "Edge.Cuts"))
 (gr_line (start 48.49153044215681 52.82214804591474) (end 48.4 52.7712812921102) (stroke (width .05) (type default)) (layer "Edge.Cuts"))
 (gr_line (start 48.4 52.7712812921102) (end 48.31018287791882 52.71744698088505) (stroke (width .05) (type default)) (layer "Edge.Cuts"))
 (gr_line (start 48.31018287791882 52.71744698088505) (end 48.22217525433727 52.66070275936814) (stroke (width .05) (type default))
  (layer "Edge.Cuts"))
 (gr_line (start 48.22217525433727 52.66070275936814) (end 48.13607137002303 52.60110939069317) (stroke (width .05) (type default))
  (layer "Edge.Cuts"))
 (gr_line (start 48.13607137002303 52.60110939069317) (end 48.05196342717209 52.53873068893195) (stroke (width .05) (type default))
  (layer "Edge.Cuts"))
 (gr_line (start 48.05196342717209 52.53873068893195) (end 47.969941490676334 52.47363345076076) (stroke (width .05) (type default))
  (layer "Edge.Cuts"))
 (gr_line (start 47.969941490676334 52.47363345076076) (end 47.89009339167978 52.40588738393273) (stroke (width .05) (type default))
  (layer "Edge.Cuts"))
 (gr_line (start 47.89009339167978 52.40588738393273) (end 47.812504633526814 52.33556503263307) (stroke (width .05) (type default))
  (layer "Edge.Cuts"))
 (gr_line (start 47.812504633526814 52.33556503263307) (end 47.737258300203045 52.26274169979695) (stroke (width .05) (type default))
  (layer "Edge.Cuts"))
 (gr_line (start 47.737258300203045 52.26274169979695) (end 47.66443496736692 52.187495366473186) (stroke (width .05) (type default))
  (layer "Edge.Cuts"))
 (gr_line (start 47.66443496736692 52.187495366473186) (end 47.59411261606727 52.109906608320216) (stroke (width .05) (type default))
  (layer "Edge.Cuts"))
 (gr_line (start 47.59411261606727 52.109906608320216) (end 47.52636654923924 52.030058509323666) (stroke (width .05) (type default))
  (layer "Edge.Cuts"))
 (gr_line (start 47.52636654923924 52.030058509323666) (end 47.5 51.99683689365963) (stroke (width .05) (type default)) (layer "Edge.Cuts"))
 (gr_line (start 47.5 51.99683689365963) (end 47.5 57.5) (stroke (width .05) (type default)) (layer "Edge.Cuts"))
 (gr_line (start 47.5 57.5) (end 47.5206484559177 57.820649217770324) (stroke (width .05) (type default)) (layer "Edge.Cuts"))
 (gr_line (start 47.5206484559177 57.820649217770324) (end 47.582252736685376 58.136001706550104) (stroke (width .05) (type default))
  (layer "Edge.Cuts"))
 (gr_line (start 47.582252736685376 58.136001706550104) (end 47.68379521568241 58.44084823276886) (stroke (width .05) (type default))
  (layer "Edge.Cuts"))
 (gr_line (start 47.68379521568241 58.44084823276886) (end 47.82359853658772 58.73015310837996) (stroke (width .05) (type default))
  (layer "Edge.Cuts"))
 (gr_line (start 47.82359853658772 58.73015310837996) (end 47.99935332123422 58.999137374206725) (stroke (width .05) (type default))
  (layer "Edge.Cuts"))
 (gr_line (start 47.99935332123422 58.999137374206725) (end 48.20815631768343 59.243357742444786) (stroke (width .05) (type default))
  (layer "Edge.Cuts"))
 (gr_line (start 48.20815631768343 59.243357742444786) (end 48.44655835836122 59.45877999428793) (stroke (width .05) (type default))
  (layer "Edge.Cuts"))
 (gr_line (start 48.44655835836122 59.45877999428793) (end 48.71062133604549 59.641845620239444) (stroke (width .05) (type default))
  (layer "Edge.Cuts"))
 (gr_line (start 48.71062133604549 59.641845620239444) (end 48.99598325653288 59.78953060229333) (stroke (width .05) (type default))
  (layer "Edge.Cuts"))
 (gr_line (start 48.99598325653288 59.78953060229333) (end 49.29793029339476 59.89939536697628) (stroke (width .05) (type default))
  (layer "Edge.Cuts"))
 (gr_line (start 49.29793029339476 59.89939536697628) (end 49.61147465456702 59.9696250840879) (stroke (width .05) (type default))
  (layer "Edge.Cuts"))
 (gr_line (start 49.61147465456702 59.9696250840879) (end 49.93143697451376 59.9990596454539) (stroke (width .05) (type default))
  (layer "Edge.Cuts"))
 (gr_line (start 49.93143697451376 59.9990596454539) (end 50.25253187094796 59.98721282848001) (stroke (width .05) (type default))
  (layer "Edge.Cuts"))
 (gr_line (start 50.25253187094796 59.98721282848001) (end 50.569455252818095 59.93428032794867) (stroke (width .05) (type default))
  (layer "Edge.Cuts"))
 (gr_line (start 50.569455252818095 59.93428032794867) (end 50.8769719373403 59.84113652338295) (stroke (width .05) (type default))
  (layer "Edge.Cuts"))
 (gr_line (start 50.8769719373403 59.84113652338295) (end 51.170002128751115 59.70932003537692) (stroke (width .05) (type default))
  (layer "Edge.Cuts"))
 (gr_line (start 51.170002128751115 59.70932003537692) (end 51.443705330258624 59.54100830948403) (stroke (width .05) (type default))
  (layer "Edge.Cuts"))
 (gr_line (start 51.443705330258624 59.54100830948403) (end 51.69356030307014 59.338981647506294) (stroke (width .05) (type default))
  (layer "Edge.Cuts"))
 (gr_line (start 51.69356030307014 59.338981647506294) (end 51.915439751672125 59.106577280342975) (stroke (width .05) (type default))
  (layer "Edge.Cuts"))
 (gr_line (start 51.915439751672125 59.106577280342975) (end 52.10567850165378 58.847634241058415) (stroke (width .05) (type default))
  (layer "Edge.Cuts"))
 (gr_line (start 52.10567850165378 58.847634241058415) (end 56.90567850165378 51.347634241058415) (stroke (width .05) (type default))
  (layer "Edge.Cuts"))
 (gr_line (start 56.90567850165378 51.347634241058415) (end 57.05888963109352 51.071175818686264) (stroke (width .05) (type default))
  (layer "Edge.Cuts"))
 (gr_line (start 57.05888963109352 51.071175818686264) (end 57.175993617117086 50.777595223377084) (stroke (width .05) (type default))
  (layer "Edge.Cuts"))
 (gr_line (start 57.175993617117086 50.777595223377084) (end 57.25511861509793 50.47158518403322) (stroke (width .05) (type default))
  (layer "Edge.Cuts"))
 (gr_line (start 57.25511861509793 50.47158518403322) (end 57.29499985423423 50.15803710757659) (stroke (width .05) (type default))
  (layer "Edge.Cuts"))
 (gr_line (start 57.29499985423423 50.15803710757659) (end 57.29499985423423 49.84196289242341) (stroke (width .05) (type default))
  (layer "Edge.Cuts"))
 (gr_line (start 57.29499985423423 49.84196289242341) (end 57.25511861509793 49.52841481596678) (stroke (width .05) (type default))
  (layer "Edge.Cuts"))
 (gr_line (start 57.25511861509793 49.52841481596678) (end 57.175993617117086 49.222404776622916) (stroke (width .05) (type default))
  (layer "Edge.Cuts"))
 (gr_line (start 57.175993617117086 49.222404776622916) (end 57.05888963109352 48.928824181313736) (stroke (width .05) (type default))
  (layer "Edge.Cuts"))
 (gr_line (start 57.05888963109352 48.928824181313736) (end 56.90567850165378 48.652365758941585) (stroke (width .05) (type default))
  (layer "Edge.Cuts"))
 (gr_line (start 56.90567850165378 48.652365758941585) (end 53.747657910476015 43.71795858522633) (stroke (width .05) (type default))
  (layer "Edge.Cuts"))
 (gr_line (start 53.747657910476015 43.71795858522633) (end 53.79748846207462 43.70104339226467) (stroke (width .05) (type default))
  (layer "Edge.Cuts"))
 (gr_line (start 53.79748846207462 43.70104339226467) (end 53.95 43.62583302491977) (stroke (width .05) (type default)) (layer "Edge.Cuts"))
 (gr_line (start 53.95 43.62583302491977) (end 54.091389857711334 43.53135934237861) (stroke (width .05) (type default)) (layer "Edge.Cuts"))
 (gr_line (start 54.091389857711334 43.53135934237861) (end 54.21923881554251 43.41923881554251) (stroke (width .05) (type default))
  (layer "Edge.Cuts"))
 (gr_line (start 54.21923881554251 43.41923881554251) (end 54.331359342378605 43.29138985771134) (stroke (width .05) (type default))
  (layer "Edge.Cuts"))
 (gr_line (start 54.331359342378605 43.29138985771134) (end 54.42583302491977 43.15) (stroke (width .05) (type default)) (layer "Edge.Cuts"))
 (gr_line (start 54.42583302491977 43.15) (end 54.50104339226467 42.997488462074614) (stroke (width .05) (type default)) (layer "Edge.Cuts"))
 (gr_line (start 54.50104339226467 42.997488462074614) (end 54.55570357417579 42.83646475863328) (stroke (width .05) (type default))
  (layer "Edge.Cuts"))
 (gr_line (start 54.55570357417579 42.83646475863328) (end 54.588878319785955 42.669684049886065) (stroke (width .05) (type default))
  (layer "Edge.Cuts"))
 (gr_line (start 54.588878319785955 42.669684049886065) (end 54.6 42.5) (stroke (width .05) (type default)) (layer "Edge.Cuts"))
 (gr_line (start 54.6 42.5) (end 54.588878319785955 42.330315950113935) (stroke (width .05) (type default)) (layer "Edge.Cuts"))
 (gr_line (start 54.588878319785955 42.330315950113935) (end 54.55570357417579 42.16353524136672) (stroke (width .05) (type default))
  (layer "Edge.Cuts"))
 (gr_line (start 54.55570357417579 42.16353524136672) (end 54.50104339226468 42.002511537925386) (stroke (width .05) (type default))
  (layer "Edge.Cuts"))
 (gr_line (start 54.50104339226468 42.002511537925386) (end 54.42583302491977 41.85) (stroke (width .05) (type default)) (layer "Edge.Cuts"))
 (gr_line (start 54.42583302491977 41.85) (end 54.331359342378605 41.70861014228866) (stroke (width .05) (type default)) (layer "Edge.Cuts"))
 (gr_line (start 54.331359342378605 41.70861014228866) (end 54.21923881554251 41.58076118445749) (stroke (width .05) (type default))
  (layer "Edge.Cuts"))
 (gr_line (start 54.21923881554251 41.58076118445749) (end 54.091389857711334 41.46864065762139) (stroke (width .05) (type default))
  (layer "Edge.Cuts"))
 (gr_line (start 54.091389857711334 41.46864065762139) (end 53.95 41.37416697508023) (stroke (width .05) (type default)) (layer "Edge.Cuts"))
 (gr_line (start 53.95 41.37416697508023) (end 53.79748846207462 41.29895660773533) (stroke (width .05) (type default)) (layer "Edge.Cuts"))
 (gr_line (start 53.79748846207462 41.29895660773533) (end 53.63646475863328 41.24429642582421) (stroke (width .05) (type default))
  (layer "Edge.Cuts"))
 (gr_line (start 53.63646475863328 41.24429642582421) (end 53.46968404988607 41.21112168021405) (stroke (width .05) (type default))
  (layer "Edge.Cuts"))
 (gr_line (start 53.46968404988607 41.21112168021405) (end 53.3 41.2) (stroke (width .05) (type default)) (layer "Edge.Cuts"))
 (gr_line (start 53.3 41.2) (end 52.13616441593116 41.2) (stroke (width .05) (type default)) (layer "Edge.Cuts"))
 (gr_line (start 52.13616441593116 41.2) (end 52.10567850165378 41.152365758941585) (stroke (width .05) (type default)) (layer "Edge.Cuts"))
 (gr_line (start 52.10567850165378 41.152365758941585) (end 51.915439751672125 40.893422719657025) (stroke (width .05) (type default))
  (layer "Edge.Cuts"))
 (gr_line (start 51.915439751672125 40.893422719657025) (end 51.69356030307014 40.661018352493706) (stroke (width .05) (type default))
  (layer "Edge.Cuts"))
 (gr_line (start 51.69356030307014 40.661018352493706) (end 51.443705330258624 40.45899169051597) (stroke (width .05) (type default))
  (layer "Edge.Cuts"))
 (gr_line (start 51.443705330258624 40.45899169051597) (end 51.170002128751115 40.29067996462308) (stroke (width .05) (type default))
  (layer "Edge.Cuts"))
 (gr_line (start 51.170002128751115 40.29067996462308) (end 50.8769719373403 40.15886347661705) (stroke (width .05) (type default))
  (layer "Edge.Cuts"))
 (gr_line (start 50.8769719373403 40.15886347661705) (end 50.569455252818095 40.06571967205133) (stroke (width .05) (type default))
  (layer "Edge.Cuts"))
 (gr_line (start 50.569455252818095 40.06571967205133) (end 50.25253187094796 40.01278717151999) (stroke (width .05) (type default))
  (layer "Edge.Cuts"))
 (gr_line (start 50.25253187094796 40.01278717151999) (end 49.93143697451376 40.0009403545461) (stroke (width .05) (type default))
  (layer "Edge.Cuts"))
 (gr_line (start 49.93143697451376 40.0009403545461) (end 49.61147465456702 40.0303749159121) (stroke (width .05) (type default))
  (layer "Edge.Cuts"))
 (gr_line (start 49.61147465456702 40.0303749159121) (end 49.29793029339476 40.10060463302372) (stroke (width .05) (type default))
  (layer "Edge.Cuts"))
 (gr_line (start 49.29793029339476 40.10060463302372) (end 48.995983256532874 40.21046939770667) (stroke (width .05) (type default))
  (layer "Edge.Cuts"))
 (gr_line (start 48.995983256532874 40.21046939770667) (end 48.71062133604549 40.358154379760556) (stroke (width .05) (type default))
  (layer "Edge.Cuts"))
 (gr_line (start 48.71062133604549 40.358154379760556) (end 48.44655835836122 40.54122000571207) (stroke (width .05) (type default))
  (layer "Edge.Cuts"))
 (gr_line (start 48.44655835836122 40.54122000571207) (end 48.20815631768343 40.756642257555214) (stroke (width .05) (type default))
  (layer "Edge.Cuts"))
 (gr_line (start 48.20815631768343 40.756642257555214) (end 47.99935332123422 41.000862625793275) (stroke (width .05) (type default))
  (layer "Edge.Cuts"))
 (gr_line (start 47.99935332123422 41.000862625793275) (end 47.869236616410625 41.2) (stroke (width .05) (type default)) (layer "Edge.Cuts"))
 (gr_line (start 47.869236616410625 41.2) (end 46.7 41.2) (stroke (width .05) (type default)) (layer "Edge.Cuts"))
 (gr_line (start 46.7 41.2) (end 46.53031595011393 41.21112168021405) (stroke (width .05) (type default)) (layer "Edge.Cuts"))
 (gr_line (start 46.53031595011393 41.21112168021405) (end 46.363535241366726 41.24429642582421) (stroke (width .05) (type default))
  (layer "Edge.Cuts")))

